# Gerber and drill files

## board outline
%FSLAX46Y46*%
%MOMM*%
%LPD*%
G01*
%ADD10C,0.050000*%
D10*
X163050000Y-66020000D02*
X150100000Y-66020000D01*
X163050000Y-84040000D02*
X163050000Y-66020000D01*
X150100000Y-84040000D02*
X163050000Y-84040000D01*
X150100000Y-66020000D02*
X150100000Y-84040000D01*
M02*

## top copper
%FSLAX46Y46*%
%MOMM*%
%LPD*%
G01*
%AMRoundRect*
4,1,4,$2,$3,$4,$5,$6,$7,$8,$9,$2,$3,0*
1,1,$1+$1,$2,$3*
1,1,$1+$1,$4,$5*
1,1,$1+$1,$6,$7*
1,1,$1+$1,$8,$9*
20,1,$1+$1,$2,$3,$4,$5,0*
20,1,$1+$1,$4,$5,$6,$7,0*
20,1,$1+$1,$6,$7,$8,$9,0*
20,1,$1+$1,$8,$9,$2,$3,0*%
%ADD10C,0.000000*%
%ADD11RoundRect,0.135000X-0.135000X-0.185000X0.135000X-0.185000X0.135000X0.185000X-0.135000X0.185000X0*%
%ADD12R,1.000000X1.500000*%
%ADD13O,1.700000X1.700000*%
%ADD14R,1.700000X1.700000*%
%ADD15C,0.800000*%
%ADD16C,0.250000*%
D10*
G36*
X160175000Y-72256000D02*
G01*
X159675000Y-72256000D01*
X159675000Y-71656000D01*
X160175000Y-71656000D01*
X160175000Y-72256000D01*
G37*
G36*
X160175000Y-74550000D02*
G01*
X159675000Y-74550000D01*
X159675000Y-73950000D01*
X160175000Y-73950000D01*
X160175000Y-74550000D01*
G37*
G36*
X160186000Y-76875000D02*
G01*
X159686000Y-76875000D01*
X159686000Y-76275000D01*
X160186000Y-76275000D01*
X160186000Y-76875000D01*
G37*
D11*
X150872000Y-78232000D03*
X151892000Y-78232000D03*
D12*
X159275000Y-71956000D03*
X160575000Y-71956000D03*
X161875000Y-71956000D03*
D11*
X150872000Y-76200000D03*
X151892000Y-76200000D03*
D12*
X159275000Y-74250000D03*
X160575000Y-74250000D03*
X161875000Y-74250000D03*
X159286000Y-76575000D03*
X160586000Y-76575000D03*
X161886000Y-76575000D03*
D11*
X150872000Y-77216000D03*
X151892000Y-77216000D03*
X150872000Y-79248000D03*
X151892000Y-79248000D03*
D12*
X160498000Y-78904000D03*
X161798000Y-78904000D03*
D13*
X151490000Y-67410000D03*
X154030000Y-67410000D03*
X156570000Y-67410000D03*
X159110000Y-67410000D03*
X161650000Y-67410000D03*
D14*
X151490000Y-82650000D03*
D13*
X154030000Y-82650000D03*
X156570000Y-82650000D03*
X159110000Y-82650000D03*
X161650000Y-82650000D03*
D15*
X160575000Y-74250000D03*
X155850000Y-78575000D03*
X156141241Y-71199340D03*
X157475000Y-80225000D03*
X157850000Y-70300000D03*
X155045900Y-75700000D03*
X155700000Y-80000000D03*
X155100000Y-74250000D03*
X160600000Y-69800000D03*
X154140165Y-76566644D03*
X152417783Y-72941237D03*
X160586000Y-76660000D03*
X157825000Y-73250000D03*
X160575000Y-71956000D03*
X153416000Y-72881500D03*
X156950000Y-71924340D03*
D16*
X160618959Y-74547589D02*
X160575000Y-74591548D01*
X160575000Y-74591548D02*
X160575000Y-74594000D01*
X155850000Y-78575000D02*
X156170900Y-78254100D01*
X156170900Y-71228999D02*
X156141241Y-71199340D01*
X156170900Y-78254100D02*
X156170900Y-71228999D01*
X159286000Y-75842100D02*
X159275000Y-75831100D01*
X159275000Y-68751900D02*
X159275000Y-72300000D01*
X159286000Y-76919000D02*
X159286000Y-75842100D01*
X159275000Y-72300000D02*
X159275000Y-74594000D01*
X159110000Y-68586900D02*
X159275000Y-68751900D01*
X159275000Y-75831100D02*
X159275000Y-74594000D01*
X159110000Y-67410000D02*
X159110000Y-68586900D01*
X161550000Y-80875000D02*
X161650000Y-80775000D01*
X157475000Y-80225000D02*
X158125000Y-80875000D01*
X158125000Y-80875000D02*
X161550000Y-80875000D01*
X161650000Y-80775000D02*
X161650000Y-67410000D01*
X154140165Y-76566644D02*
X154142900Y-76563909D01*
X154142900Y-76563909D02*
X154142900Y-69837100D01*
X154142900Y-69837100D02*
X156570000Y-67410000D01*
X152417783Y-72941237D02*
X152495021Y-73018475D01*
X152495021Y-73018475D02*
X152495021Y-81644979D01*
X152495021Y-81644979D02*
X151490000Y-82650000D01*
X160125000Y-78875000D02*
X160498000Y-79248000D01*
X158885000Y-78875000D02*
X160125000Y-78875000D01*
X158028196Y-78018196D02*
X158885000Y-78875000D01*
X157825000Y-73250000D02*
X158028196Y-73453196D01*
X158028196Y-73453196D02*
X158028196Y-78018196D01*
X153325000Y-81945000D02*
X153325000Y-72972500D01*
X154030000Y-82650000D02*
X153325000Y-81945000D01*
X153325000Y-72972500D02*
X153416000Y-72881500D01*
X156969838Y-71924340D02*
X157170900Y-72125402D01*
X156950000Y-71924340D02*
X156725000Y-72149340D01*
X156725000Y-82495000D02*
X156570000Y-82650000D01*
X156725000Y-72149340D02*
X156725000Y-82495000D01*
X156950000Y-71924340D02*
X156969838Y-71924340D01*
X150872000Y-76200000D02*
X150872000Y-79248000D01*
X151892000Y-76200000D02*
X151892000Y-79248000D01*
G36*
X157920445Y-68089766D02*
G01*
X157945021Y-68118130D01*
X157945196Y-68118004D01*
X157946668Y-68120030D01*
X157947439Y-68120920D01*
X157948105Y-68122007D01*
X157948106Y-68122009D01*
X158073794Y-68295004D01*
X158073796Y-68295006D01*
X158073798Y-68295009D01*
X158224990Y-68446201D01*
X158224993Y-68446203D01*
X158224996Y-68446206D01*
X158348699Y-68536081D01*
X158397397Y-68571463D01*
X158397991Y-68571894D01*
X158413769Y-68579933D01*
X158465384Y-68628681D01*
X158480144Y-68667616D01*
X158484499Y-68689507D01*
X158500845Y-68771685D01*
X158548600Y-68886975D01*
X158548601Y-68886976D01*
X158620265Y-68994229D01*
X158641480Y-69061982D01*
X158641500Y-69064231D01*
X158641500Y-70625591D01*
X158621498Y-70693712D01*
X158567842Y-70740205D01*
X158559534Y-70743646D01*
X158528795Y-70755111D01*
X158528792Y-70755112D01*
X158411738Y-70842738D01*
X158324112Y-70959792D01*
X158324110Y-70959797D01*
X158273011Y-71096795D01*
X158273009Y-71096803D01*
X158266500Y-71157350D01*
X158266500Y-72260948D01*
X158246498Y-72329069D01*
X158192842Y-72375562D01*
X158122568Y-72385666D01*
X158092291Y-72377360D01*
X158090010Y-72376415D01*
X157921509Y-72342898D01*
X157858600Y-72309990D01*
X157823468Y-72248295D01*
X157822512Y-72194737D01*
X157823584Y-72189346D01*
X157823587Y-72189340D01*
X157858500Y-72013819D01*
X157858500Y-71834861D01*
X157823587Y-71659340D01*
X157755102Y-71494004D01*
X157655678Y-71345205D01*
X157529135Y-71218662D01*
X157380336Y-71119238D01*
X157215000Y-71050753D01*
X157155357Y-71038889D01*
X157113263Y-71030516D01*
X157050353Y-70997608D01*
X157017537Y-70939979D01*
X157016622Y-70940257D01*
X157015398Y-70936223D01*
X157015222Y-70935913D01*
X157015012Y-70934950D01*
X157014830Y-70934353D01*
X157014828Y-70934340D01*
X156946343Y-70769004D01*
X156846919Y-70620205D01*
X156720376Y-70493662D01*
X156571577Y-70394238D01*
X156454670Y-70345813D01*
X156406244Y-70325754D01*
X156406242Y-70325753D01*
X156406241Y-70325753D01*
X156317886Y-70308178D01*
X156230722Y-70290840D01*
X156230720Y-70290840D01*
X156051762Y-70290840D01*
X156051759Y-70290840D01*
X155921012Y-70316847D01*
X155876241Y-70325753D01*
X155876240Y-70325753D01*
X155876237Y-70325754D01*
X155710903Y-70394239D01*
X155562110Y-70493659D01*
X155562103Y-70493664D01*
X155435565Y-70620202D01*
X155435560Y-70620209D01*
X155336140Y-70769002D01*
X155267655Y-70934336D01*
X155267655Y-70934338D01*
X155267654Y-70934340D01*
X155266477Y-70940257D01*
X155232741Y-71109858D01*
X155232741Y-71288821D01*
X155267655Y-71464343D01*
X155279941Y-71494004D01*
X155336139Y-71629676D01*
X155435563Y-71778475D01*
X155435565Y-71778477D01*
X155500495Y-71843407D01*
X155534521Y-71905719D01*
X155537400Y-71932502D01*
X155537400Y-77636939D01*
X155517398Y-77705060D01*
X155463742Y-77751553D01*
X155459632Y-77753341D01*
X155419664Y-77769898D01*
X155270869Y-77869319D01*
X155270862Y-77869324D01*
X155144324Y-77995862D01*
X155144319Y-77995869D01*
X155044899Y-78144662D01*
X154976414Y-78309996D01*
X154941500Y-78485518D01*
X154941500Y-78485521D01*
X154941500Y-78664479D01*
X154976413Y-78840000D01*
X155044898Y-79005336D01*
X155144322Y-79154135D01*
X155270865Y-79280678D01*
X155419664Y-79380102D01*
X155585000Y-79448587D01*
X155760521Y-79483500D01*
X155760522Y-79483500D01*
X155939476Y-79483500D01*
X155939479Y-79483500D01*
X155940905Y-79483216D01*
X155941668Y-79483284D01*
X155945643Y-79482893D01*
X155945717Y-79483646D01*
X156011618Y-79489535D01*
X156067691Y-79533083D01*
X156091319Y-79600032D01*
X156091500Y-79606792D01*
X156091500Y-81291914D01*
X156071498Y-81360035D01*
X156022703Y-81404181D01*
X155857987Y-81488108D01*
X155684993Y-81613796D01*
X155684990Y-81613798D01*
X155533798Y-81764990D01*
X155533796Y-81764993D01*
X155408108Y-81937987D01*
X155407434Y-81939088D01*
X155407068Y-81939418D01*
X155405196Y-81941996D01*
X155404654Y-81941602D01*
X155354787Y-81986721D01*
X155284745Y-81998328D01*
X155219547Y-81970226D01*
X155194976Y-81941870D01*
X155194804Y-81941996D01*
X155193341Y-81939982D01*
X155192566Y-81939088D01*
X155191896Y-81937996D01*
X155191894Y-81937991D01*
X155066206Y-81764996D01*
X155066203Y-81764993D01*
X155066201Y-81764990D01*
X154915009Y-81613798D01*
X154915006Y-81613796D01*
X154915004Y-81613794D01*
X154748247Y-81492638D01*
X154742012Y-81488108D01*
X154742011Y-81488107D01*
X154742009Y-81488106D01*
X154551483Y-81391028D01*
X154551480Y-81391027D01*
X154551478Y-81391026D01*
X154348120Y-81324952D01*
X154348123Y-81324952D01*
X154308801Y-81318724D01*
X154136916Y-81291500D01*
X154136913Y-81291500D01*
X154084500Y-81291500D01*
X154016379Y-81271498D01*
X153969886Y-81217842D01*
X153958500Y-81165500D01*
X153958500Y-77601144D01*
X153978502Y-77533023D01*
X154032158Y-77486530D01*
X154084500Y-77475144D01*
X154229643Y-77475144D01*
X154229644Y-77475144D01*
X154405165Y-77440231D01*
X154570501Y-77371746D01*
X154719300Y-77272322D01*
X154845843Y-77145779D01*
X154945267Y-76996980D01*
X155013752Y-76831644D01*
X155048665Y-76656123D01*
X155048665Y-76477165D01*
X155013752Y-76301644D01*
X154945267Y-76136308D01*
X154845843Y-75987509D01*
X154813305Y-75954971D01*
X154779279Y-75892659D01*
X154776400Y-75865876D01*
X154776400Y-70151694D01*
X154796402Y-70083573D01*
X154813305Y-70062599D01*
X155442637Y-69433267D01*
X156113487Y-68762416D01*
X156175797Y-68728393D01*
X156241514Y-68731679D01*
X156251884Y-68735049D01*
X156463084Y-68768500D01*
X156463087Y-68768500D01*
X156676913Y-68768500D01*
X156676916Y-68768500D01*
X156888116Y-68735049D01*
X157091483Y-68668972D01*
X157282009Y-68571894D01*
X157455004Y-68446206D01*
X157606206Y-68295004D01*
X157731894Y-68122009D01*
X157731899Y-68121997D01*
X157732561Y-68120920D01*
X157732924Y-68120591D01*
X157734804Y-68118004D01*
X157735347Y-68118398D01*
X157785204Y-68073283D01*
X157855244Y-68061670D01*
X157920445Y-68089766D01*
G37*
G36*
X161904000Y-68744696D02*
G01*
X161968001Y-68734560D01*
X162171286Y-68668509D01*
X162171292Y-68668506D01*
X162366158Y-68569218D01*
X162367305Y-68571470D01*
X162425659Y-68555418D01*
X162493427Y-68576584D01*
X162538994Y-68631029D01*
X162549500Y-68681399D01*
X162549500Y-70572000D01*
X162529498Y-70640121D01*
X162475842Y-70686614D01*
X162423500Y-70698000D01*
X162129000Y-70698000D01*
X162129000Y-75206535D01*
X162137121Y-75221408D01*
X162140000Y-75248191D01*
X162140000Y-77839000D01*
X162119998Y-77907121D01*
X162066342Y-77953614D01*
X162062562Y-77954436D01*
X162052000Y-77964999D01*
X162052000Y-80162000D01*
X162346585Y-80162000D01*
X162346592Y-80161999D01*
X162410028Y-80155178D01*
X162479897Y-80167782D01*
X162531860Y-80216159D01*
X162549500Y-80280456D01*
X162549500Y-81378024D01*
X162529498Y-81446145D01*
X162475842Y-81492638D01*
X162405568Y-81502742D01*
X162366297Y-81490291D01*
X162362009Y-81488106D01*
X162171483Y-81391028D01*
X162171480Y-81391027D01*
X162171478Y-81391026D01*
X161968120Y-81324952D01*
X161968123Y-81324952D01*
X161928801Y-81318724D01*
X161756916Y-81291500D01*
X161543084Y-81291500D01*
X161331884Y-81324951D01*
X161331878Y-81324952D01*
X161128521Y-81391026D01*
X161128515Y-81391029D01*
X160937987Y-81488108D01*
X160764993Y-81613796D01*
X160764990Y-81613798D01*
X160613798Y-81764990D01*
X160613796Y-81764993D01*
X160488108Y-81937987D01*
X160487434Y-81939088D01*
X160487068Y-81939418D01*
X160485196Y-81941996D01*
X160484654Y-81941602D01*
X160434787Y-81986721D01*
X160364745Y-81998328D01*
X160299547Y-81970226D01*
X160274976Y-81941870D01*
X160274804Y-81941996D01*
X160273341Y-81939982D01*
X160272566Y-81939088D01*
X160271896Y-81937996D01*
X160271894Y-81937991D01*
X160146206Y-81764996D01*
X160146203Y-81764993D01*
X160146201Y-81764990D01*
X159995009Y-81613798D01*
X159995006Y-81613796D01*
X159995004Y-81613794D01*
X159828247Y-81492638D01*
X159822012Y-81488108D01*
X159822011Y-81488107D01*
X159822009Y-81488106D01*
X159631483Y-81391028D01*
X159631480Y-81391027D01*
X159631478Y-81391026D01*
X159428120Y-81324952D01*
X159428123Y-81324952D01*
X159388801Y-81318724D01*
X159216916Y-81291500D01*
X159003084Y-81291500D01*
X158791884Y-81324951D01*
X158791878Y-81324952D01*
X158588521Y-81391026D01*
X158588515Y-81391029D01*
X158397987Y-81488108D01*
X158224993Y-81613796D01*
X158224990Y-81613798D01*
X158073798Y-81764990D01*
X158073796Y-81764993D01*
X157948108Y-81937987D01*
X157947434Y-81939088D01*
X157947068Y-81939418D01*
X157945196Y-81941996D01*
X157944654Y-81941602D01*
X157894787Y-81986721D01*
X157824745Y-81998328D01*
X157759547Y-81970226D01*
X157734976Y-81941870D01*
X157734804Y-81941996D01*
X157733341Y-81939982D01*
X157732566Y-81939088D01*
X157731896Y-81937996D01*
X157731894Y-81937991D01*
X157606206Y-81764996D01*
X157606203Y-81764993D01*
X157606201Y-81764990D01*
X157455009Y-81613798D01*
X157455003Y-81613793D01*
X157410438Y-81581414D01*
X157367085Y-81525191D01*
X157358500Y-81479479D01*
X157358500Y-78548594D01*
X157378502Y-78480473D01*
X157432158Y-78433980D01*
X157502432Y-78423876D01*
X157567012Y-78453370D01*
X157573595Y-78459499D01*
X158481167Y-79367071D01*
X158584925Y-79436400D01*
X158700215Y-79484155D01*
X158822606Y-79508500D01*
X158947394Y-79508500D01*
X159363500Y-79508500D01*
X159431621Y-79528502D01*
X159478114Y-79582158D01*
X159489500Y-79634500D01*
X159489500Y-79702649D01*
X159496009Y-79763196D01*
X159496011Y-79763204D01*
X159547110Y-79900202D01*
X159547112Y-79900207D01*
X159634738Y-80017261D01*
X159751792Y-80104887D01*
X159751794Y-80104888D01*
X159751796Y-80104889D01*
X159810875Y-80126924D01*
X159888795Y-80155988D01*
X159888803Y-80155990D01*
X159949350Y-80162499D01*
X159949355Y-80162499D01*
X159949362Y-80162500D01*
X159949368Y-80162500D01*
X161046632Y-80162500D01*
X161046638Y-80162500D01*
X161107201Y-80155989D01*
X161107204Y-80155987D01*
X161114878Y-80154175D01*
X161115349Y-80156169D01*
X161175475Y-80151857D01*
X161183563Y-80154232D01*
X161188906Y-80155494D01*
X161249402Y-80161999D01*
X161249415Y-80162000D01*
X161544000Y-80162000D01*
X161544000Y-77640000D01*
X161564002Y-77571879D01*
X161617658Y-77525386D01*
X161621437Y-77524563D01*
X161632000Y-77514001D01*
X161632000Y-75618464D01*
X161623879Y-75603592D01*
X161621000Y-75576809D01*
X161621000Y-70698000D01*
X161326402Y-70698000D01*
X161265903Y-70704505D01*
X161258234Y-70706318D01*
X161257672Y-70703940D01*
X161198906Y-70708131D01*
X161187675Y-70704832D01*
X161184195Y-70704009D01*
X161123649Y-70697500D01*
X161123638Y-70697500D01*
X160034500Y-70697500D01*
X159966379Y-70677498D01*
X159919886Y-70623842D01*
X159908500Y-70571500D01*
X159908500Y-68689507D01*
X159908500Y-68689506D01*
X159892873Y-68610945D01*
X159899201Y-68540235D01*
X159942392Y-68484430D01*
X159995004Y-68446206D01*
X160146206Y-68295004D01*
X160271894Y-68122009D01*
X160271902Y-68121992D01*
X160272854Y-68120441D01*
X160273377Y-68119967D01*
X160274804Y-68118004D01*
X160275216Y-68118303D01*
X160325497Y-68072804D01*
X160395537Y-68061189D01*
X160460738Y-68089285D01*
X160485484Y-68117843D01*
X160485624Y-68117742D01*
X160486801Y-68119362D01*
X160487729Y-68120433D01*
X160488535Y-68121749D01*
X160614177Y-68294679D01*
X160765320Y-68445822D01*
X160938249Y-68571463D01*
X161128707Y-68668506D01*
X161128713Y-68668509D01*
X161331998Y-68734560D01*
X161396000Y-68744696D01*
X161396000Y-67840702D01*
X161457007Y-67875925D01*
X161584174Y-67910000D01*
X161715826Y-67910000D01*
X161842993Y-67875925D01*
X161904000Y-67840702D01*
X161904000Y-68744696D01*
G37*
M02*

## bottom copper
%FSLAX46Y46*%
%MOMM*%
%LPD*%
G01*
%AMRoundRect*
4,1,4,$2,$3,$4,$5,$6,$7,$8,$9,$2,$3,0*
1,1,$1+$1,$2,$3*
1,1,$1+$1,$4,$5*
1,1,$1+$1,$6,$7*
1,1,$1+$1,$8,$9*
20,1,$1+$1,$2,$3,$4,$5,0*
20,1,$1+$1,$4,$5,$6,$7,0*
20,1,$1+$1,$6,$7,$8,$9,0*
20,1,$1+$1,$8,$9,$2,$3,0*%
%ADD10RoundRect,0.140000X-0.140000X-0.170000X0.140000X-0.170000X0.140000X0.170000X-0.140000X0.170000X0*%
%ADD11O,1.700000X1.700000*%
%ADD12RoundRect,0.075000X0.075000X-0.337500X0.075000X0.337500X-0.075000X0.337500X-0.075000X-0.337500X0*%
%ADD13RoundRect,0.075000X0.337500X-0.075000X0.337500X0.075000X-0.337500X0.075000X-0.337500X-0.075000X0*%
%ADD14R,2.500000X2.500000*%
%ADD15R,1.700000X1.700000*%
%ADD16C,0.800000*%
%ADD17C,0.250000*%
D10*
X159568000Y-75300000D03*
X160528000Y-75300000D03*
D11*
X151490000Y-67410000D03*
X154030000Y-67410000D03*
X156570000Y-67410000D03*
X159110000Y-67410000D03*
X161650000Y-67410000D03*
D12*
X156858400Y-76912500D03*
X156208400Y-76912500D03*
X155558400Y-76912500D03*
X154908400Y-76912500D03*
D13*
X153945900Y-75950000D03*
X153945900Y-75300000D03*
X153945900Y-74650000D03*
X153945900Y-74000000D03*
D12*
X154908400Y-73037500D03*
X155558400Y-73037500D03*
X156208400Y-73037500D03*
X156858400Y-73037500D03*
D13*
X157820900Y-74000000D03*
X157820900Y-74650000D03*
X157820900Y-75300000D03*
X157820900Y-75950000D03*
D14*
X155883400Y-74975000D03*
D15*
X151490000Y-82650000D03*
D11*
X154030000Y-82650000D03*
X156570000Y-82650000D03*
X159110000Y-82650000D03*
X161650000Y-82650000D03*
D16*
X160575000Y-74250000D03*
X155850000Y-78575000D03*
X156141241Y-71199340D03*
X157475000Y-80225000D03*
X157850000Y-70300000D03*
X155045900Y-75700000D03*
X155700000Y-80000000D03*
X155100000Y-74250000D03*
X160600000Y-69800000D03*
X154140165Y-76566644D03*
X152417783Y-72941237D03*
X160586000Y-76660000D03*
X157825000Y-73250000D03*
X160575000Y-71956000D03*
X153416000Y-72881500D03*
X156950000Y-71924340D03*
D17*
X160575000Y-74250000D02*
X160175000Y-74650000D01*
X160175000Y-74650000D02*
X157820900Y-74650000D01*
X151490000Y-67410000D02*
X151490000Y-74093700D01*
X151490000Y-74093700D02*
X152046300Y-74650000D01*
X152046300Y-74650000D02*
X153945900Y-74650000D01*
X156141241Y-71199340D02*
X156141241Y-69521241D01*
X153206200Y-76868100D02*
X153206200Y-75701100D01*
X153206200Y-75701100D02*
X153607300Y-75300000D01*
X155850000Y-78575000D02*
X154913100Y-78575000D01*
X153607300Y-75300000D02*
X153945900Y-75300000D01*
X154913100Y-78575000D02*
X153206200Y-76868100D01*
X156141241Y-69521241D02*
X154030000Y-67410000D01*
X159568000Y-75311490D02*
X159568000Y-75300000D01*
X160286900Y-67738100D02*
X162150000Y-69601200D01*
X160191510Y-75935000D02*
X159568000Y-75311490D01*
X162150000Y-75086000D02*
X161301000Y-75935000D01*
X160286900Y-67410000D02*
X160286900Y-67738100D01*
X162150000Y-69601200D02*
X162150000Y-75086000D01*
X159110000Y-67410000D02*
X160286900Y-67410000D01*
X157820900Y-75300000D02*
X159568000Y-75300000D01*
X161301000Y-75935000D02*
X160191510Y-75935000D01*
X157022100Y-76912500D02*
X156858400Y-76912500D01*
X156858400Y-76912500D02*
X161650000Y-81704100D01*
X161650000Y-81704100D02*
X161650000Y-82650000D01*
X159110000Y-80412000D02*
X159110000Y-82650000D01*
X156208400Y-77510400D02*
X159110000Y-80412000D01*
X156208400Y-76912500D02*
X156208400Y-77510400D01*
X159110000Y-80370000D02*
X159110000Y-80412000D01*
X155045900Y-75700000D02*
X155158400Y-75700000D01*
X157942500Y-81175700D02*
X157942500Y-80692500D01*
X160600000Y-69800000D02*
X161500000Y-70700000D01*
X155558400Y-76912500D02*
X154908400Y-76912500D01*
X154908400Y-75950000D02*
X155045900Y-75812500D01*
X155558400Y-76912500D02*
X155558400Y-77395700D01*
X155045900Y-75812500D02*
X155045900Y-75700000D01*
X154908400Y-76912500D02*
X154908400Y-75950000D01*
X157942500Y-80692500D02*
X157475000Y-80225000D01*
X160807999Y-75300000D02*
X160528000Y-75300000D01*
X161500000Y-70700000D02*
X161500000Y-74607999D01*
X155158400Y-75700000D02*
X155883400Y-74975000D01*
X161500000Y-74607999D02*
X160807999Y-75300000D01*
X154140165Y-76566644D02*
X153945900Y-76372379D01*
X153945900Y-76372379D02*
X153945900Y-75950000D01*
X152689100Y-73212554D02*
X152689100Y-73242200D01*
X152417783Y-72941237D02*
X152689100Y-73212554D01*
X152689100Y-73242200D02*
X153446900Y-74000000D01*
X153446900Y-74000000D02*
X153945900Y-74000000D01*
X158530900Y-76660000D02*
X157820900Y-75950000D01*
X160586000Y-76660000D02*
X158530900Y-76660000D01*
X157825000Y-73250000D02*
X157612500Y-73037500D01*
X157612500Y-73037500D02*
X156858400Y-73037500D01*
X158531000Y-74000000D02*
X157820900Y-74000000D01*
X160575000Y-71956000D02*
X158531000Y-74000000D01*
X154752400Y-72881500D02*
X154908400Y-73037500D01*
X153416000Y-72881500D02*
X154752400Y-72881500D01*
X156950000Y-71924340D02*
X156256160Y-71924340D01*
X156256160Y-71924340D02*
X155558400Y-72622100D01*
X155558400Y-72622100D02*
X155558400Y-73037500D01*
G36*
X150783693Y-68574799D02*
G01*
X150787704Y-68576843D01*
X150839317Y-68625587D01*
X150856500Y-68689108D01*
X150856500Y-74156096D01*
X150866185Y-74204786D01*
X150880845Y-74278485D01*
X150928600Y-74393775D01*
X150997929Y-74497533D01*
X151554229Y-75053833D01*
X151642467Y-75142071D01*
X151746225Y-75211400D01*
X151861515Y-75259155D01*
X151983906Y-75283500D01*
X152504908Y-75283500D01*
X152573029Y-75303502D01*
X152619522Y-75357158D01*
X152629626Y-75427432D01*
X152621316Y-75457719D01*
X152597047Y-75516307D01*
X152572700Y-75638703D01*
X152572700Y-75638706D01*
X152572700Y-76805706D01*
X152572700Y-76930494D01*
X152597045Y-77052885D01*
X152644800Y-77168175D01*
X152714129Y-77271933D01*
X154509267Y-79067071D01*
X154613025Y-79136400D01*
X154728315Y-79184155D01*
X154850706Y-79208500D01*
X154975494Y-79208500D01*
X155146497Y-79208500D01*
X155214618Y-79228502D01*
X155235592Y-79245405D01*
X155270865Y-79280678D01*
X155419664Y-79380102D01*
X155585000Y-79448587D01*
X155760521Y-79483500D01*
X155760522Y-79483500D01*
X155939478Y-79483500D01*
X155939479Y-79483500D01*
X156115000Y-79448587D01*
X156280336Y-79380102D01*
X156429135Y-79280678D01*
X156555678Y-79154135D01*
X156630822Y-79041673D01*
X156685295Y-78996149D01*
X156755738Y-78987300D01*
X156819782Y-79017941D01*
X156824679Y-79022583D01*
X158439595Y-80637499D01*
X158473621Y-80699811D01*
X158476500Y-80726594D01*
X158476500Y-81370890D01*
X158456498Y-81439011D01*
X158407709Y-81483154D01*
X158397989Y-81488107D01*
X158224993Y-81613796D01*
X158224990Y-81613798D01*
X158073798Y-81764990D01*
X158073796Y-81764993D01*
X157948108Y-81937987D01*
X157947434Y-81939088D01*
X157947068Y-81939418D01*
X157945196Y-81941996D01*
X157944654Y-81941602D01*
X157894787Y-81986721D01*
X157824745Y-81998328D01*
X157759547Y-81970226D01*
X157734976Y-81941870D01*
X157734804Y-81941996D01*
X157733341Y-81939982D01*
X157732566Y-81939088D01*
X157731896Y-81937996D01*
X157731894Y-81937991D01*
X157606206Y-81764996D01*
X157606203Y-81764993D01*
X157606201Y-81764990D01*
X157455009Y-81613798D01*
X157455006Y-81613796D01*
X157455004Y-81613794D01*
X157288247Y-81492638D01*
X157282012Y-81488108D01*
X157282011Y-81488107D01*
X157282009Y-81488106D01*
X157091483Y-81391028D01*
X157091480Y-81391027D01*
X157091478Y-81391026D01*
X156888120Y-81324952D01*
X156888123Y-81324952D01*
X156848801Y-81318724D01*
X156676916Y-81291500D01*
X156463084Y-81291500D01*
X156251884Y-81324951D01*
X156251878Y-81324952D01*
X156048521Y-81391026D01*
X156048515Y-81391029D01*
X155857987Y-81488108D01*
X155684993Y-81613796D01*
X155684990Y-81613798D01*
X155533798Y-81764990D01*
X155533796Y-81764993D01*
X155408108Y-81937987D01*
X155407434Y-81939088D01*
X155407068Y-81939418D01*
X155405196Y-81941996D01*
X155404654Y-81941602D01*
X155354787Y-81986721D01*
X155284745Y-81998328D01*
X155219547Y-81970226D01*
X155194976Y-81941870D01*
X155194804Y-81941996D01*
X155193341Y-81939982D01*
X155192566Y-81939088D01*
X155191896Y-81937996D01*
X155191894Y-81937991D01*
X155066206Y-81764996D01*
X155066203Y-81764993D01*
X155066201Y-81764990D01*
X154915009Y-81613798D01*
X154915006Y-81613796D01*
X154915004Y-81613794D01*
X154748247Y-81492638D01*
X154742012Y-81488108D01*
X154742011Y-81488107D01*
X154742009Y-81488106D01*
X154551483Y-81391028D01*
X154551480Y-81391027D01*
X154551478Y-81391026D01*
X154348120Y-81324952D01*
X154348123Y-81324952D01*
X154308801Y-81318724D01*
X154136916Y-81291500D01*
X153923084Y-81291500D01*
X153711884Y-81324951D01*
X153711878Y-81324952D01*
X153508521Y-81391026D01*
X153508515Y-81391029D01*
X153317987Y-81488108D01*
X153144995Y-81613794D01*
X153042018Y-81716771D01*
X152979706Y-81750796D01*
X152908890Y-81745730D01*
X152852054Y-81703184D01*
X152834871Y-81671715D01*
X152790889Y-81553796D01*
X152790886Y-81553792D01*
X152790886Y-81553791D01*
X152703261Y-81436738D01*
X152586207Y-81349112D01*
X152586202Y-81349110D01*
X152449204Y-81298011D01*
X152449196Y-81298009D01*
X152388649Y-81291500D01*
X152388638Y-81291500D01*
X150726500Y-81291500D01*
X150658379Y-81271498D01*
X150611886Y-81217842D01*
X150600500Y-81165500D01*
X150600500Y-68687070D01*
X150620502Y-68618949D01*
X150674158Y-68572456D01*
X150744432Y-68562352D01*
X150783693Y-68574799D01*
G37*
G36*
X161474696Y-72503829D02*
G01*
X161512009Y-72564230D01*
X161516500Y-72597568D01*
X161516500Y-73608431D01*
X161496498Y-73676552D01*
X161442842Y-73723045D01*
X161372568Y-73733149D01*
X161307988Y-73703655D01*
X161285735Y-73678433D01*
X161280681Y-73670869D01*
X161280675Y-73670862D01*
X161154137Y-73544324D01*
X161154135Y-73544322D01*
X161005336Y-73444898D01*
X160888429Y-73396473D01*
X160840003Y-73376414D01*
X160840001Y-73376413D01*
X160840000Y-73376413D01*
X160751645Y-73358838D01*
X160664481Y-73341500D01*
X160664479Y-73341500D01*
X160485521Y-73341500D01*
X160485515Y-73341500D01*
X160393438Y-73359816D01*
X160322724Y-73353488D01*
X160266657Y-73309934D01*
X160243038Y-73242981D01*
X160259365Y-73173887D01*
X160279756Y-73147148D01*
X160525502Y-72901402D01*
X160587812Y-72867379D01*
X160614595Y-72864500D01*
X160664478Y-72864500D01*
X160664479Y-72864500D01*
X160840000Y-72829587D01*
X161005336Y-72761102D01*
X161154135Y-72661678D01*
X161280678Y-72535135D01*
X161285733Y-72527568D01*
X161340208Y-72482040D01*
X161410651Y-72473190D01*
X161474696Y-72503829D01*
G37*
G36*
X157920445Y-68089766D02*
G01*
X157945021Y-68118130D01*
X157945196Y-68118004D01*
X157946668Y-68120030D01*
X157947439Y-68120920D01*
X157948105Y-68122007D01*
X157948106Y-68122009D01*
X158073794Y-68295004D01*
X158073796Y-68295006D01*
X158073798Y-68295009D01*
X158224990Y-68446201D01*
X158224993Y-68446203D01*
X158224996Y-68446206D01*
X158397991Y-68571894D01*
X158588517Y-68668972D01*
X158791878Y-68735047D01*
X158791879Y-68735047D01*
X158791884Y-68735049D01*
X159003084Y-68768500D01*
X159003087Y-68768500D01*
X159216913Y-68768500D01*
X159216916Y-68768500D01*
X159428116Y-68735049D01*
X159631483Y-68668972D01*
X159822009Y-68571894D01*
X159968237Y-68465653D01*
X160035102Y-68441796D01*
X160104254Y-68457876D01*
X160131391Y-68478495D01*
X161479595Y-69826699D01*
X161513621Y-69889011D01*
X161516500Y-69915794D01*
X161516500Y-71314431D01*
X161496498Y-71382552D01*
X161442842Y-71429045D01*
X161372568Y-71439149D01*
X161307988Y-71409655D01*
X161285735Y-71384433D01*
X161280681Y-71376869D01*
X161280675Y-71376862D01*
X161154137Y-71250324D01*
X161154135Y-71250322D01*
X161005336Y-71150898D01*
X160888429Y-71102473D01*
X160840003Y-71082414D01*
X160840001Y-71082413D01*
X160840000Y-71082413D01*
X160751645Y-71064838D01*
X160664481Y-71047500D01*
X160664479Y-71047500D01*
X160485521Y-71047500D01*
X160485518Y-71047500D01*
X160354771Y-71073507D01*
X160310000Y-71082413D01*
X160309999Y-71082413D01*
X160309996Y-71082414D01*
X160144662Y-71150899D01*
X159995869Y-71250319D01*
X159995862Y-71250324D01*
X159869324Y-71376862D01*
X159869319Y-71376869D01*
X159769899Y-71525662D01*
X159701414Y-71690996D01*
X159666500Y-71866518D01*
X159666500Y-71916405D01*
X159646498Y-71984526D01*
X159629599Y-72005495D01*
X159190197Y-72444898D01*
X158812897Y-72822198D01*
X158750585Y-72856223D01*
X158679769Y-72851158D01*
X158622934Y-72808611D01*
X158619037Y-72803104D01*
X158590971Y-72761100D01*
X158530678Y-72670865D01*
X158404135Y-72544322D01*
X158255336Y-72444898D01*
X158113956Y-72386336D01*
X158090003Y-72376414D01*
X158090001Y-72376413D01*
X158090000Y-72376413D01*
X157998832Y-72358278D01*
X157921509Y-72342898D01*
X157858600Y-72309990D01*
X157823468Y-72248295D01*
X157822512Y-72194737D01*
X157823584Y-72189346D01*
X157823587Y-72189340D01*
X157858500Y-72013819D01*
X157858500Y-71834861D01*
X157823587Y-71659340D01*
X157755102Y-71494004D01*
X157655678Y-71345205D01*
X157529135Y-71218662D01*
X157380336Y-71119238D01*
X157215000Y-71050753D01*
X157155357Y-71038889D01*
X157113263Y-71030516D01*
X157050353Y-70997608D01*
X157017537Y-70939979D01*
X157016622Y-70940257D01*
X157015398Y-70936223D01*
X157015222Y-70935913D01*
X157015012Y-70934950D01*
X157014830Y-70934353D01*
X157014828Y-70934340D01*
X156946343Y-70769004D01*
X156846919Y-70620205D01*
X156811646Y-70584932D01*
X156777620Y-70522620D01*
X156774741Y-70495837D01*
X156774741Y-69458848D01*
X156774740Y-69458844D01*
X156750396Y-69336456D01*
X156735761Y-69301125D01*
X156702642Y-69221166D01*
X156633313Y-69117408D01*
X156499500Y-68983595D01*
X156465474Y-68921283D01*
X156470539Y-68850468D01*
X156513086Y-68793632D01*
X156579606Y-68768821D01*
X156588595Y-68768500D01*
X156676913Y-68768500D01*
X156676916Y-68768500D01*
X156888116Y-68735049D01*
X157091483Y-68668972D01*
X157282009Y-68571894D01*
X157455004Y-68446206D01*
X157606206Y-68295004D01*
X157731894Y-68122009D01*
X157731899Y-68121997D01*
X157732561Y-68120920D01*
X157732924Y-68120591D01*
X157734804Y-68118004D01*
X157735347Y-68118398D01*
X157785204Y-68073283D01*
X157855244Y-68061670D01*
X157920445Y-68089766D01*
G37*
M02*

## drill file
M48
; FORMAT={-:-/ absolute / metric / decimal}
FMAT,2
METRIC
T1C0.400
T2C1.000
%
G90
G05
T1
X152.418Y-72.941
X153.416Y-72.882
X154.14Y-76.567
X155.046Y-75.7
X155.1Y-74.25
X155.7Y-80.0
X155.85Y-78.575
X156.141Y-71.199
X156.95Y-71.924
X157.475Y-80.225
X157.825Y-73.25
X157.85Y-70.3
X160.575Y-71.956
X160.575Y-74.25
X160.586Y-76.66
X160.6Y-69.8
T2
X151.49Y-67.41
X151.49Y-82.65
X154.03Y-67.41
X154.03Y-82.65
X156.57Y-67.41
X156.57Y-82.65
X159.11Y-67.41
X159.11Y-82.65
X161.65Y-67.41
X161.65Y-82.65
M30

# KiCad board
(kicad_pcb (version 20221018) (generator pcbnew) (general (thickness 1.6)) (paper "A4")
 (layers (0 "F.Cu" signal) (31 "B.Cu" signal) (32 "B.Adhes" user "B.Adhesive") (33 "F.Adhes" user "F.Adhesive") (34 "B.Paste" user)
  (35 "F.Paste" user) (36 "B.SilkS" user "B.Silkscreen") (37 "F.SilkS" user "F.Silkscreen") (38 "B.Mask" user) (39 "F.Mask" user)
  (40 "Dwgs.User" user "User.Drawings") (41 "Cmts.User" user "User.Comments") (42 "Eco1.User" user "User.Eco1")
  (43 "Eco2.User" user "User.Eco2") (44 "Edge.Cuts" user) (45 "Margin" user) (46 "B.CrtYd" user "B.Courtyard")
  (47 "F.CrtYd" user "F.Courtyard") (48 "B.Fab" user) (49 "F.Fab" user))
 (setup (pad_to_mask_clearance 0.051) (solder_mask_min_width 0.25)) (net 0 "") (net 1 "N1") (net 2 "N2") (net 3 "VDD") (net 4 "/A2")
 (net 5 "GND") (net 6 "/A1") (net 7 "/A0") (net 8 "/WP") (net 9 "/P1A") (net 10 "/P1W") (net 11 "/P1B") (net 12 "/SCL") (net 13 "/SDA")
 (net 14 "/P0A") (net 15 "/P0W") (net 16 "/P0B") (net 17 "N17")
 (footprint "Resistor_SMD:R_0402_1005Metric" (layer "F.Cu") (at 151.382 78.232)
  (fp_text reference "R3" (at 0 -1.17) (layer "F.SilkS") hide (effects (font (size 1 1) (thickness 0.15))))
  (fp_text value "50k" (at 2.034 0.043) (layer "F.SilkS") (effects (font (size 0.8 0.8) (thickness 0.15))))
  (pad "1" smd roundrect (at -0.51 0) (size 0.54 0.64) (layers "F.Cu" "F.Paste" "F.Mask") (roundrect_rratio 0.25) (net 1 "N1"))
  (pad "2" smd roundrect (at 0.51 0) (size 0.54 0.64) (layers "F.Cu" "F.Paste" "F.Mask") (roundrect_rratio 0.25) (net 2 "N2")))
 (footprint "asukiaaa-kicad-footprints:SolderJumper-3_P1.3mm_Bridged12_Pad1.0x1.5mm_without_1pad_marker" (layer "F.Cu") (at 160.575 71.956)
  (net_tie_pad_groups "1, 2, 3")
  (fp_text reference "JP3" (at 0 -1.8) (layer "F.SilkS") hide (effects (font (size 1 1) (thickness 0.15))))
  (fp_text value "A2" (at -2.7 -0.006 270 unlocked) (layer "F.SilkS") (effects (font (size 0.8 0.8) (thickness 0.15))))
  (fp_poly (pts (xy -0.9 -0.3) (xy -0.4 -0.3) (xy -0.4 0.3) (xy -0.9 0.3)) (stroke (width 0) (type solid)) (fill solid) (layer "F.Cu"))
  (pad "1" smd rect (at -1.3 0) (size 1 1.5) (layers "F.Cu" "F.Mask") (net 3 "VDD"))
  (pad "2" smd rect (at 0 0) (size 1 1.5) (layers "F.Cu" "F.Mask") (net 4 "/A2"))
  (pad "3" smd rect (at 1.3 0) (size 1 1.5) (layers "F.Cu" "F.Mask") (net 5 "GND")))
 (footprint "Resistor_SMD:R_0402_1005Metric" (layer "F.Cu") (at 151.382 76.2)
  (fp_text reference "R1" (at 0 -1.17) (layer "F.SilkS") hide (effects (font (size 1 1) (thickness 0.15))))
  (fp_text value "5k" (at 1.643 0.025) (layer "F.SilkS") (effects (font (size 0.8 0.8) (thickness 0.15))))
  (pad "1" smd roundrect (at -0.51 0) (size 0.54 0.64) (layers "F.Cu" "F.Paste" "F.Mask") (roundrect_rratio 0.25) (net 1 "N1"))
  (pad "2" smd roundrect (at 0.51 0) (size 0.54 0.64) (layers "F.Cu" "F.Paste" "F.Mask") (roundrect_rratio 0.25) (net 2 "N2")))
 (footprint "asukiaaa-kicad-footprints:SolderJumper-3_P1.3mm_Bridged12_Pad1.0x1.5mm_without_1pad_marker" (layer "F.Cu") (at 160.575 74.25)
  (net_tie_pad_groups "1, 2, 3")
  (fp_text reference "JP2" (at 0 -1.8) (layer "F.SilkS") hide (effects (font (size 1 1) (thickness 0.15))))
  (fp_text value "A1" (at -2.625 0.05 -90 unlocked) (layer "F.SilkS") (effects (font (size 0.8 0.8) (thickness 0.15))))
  (fp_poly (pts (xy -0.9 -0.3) (xy -0.4 -0.3) (xy -0.4 0.3) (xy -0.9 0.3)) (stroke (width 0) (type solid)) (fill solid) (layer "F.Cu"))
  (pad "1" smd rect (at -1.3 0) (size 1 1.5) (layers "F.Cu" "F.Mask") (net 3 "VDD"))
  (pad "2" smd rect (at 0 0) (size 1 1.5) (layers "F.Cu" "F.Mask") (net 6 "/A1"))
  (pad "3" smd rect (at 1.3 0) (size 1 1.5) (layers "F.Cu" "F.Mask") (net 5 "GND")))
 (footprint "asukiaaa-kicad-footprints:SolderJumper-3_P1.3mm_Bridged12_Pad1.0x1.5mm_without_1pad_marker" (layer "F.Cu") (at 160.586 76.575)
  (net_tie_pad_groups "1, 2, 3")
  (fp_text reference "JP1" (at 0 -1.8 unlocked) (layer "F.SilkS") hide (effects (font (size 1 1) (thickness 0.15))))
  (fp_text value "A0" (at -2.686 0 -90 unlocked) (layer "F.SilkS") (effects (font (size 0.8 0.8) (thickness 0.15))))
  (fp_poly (pts (xy -0.9 -0.3) (xy -0.4 -0.3) (xy -0.4 0.3) (xy -0.9 0.3)) (stroke (width 0) (type solid)) (fill solid) (layer "F.Cu"))
  (pad "1" smd rect (at -1.3 0) (size 1 1.5) (layers "F.Cu" "F.Mask") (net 3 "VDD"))
  (pad "2" smd rect (at 0 0) (size 1 1.5) (layers "F.Cu" "F.Mask") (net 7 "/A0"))
  (pad "3" smd rect (at 1.3 0) (size 1 1.5) (layers "F.Cu" "F.Mask") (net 5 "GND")))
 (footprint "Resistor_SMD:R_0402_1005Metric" (layer "F.Cu") (at 151.382 77.216)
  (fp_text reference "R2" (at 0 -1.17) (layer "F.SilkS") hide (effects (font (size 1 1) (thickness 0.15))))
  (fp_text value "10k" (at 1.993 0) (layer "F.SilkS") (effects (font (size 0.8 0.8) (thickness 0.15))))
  (pad "1" smd roundrect (at -0.51 0) (size 0.54 0.64) (layers "F.Cu" "F.Paste" "F.Mask") (roundrect_rratio 0.25) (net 1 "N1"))
  (pad "2" smd roundrect (at 0.51 0) (size 0.54 0.64) (layers "F.Cu" "F.Paste" "F.Mask") (roundrect_rratio 0.25) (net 2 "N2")))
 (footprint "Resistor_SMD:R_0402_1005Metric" (layer "F.Cu") (at 151.382 79.248)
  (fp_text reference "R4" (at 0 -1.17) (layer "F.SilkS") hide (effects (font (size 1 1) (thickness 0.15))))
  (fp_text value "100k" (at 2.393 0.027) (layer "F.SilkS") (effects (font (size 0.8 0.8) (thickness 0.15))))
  (pad "1" smd roundrect (at -0.51 0) (size 0.54 0.64) (layers "F.Cu" "F.Paste" "F.Mask") (roundrect_rratio 0.25) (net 1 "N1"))
  (pad "2" smd roundrect (at 0.51 0) (size 0.54 0.64) (layers "F.Cu" "F.Paste" "F.Mask") (roundrect_rratio 0.25) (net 2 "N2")))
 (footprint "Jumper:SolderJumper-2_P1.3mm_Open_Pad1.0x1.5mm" (layer "F.Cu") (at 161.148 78.904)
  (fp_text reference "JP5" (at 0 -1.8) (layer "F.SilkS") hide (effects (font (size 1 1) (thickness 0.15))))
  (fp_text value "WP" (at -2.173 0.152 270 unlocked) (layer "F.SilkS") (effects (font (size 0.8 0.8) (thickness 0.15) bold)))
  (pad "1" smd rect (at -0.65 0) (size 1 1.5) (layers "F.Cu" "F.Mask") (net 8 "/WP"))
  (pad "2" smd rect (at 0.65 0) (size 1 1.5) (layers "F.Cu" "F.Mask") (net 5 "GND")))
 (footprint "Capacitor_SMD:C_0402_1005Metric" (layer "B.Cu") (at 160.048 75.3)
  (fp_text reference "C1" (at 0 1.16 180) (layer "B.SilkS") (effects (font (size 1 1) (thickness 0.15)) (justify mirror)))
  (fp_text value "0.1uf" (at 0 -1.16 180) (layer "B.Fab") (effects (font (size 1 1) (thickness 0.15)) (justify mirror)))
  (pad "1" smd roundrect (at -0.48 0) (size 0.56 0.62) (layers "B.Cu" "B.Paste" "B.Mask") (roundrect_rratio 0.25) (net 3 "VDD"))
  (pad "2" smd roundrect (at 0.48 0) (size 0.56 0.62) (layers "B.Cu" "B.Paste" "B.Mask") (roundrect_rratio 0.25) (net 5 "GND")))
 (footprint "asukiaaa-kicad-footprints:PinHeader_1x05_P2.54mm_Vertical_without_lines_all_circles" (layer "B.Cu") (at 151.49 67.41 -90)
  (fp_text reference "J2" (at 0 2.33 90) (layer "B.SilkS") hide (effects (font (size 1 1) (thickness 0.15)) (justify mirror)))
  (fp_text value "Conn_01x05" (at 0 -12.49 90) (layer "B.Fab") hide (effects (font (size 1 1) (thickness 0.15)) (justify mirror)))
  (pad "1" thru_hole oval (at 0 0 270) (size 1.7 1.7) (drill 1) (layers "*.Cu" "*.Mask") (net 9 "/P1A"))
  (pad "2" thru_hole oval (at 0 -2.54 270) (size 1.7 1.7) (drill 1) (layers "*.Cu" "*.Mask") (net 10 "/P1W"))
  (pad "3" thru_hole oval (at 0 -5.08 270) (size 1.7 1.7) (drill 1) (layers "*.Cu" "*.Mask") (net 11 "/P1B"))
  (pad "4" thru_hole oval (at 0 -7.62 270) (size 1.7 1.7) (drill 1) (layers "*.Cu" "*.Mask") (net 3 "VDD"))
  (pad "5" thru_hole oval (at 0 -10.16 270) (size 1.7 1.7) (drill 1) (layers "*.Cu" "*.Mask") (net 5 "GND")))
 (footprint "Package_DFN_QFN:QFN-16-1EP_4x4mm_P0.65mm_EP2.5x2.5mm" (layer "B.Cu") (at 155.8834 74.975 90)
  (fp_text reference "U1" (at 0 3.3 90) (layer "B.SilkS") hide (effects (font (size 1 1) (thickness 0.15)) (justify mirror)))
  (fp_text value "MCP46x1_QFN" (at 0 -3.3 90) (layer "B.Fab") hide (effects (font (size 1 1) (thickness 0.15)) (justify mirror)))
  (pad "" smd roundrect (at -0.625 -0.625 90) (size 1.01 1.01) (layers "B.Paste") (roundrect_rratio 0.247525))
  (pad "" smd roundrect (at -0.625 0.625 90) (size 1.01 1.01) (layers "B.Paste") (roundrect_rratio 0.247525))
  (pad "" smd roundrect (at 0.625 -0.625 90) (size 1.01 1.01) (layers "B.Paste") (roundrect_rratio 0.247525))
  (pad "" smd roundrect (at 0.625 0.625 90) (size 1.01 1.01) (layers "B.Paste") (roundrect_rratio 0.247525))
  (pad "1" smd roundrect (at -1.9375 0.975 90) (size 0.825 0.3) (layers "B.Cu" "B.Paste" "B.Mask") (roundrect_rratio 0.25) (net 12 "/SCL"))
  (pad "2" smd roundrect (at -1.9375 0.325 90) (size 0.825 0.3) (layers "B.Cu" "B.Paste" "B.Mask") (roundrect_rratio 0.25) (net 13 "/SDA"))
  (pad "3" smd roundrect (at -1.9375 -0.325 90) (size 0.825 0.3) (layers "B.Cu" "B.Paste" "B.Mask") (roundrect_rratio 0.25) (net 5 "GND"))
  (pad "4" smd roundrect (at -1.9375 -0.975 90) (size 0.825 0.3) (layers "B.Cu" "B.Paste" "B.Mask") (roundrect_rratio 0.25) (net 5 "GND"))
  (pad "5" smd roundrect (at -0.975 -1.9375 90) (size 0.3 0.825) (layers "B.Cu" "B.Paste" "B.Mask") (roundrect_rratio 0.25) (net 11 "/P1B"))
  (pad "6" smd roundrect (at -0.325 -1.9375 90) (size 0.3 0.825) (layers "B.Cu" "B.Paste" "B.Mask") (roundrect_rratio 0.25) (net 10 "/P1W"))
  (pad "7" smd roundrect (at 0.325 -1.9375 90) (size 0.3 0.825) (layers "B.Cu" "B.Paste" "B.Mask") (roundrect_rratio 0.25) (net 9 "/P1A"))
  (pad "8" smd roundrect (at 0.975 -1.9375 90) (size 0.3 0.825) (layers "B.Cu" "B.Paste" "B.Mask") (roundrect_rratio 0.25) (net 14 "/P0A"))
  (pad "9" smd roundrect (at 1.9375 -0.975 90) (size 0.825 0.3) (layers "B.Cu" "B.Paste" "B.Mask") (roundrect_rratio 0.25) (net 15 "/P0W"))
  (pad "10" smd roundrect (at 1.9375 -0.325 90) (size 0.825 0.3) (layers "B.Cu" "B.Paste" "B.Mask") (roundrect_rratio 0.25) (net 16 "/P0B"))
  (pad "11" smd roundrect (at 1.9375 0.325 90) (size 0.825 0.3) (layers "B.Cu" "B.Paste" "B.Mask") (roundrect_rratio 0.25) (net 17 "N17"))
  (pad "12" smd roundrect (at 1.9375 0.975 90) (size 0.825 0.3) (layers "B.Cu" "B.Paste" "B.Mask") (roundrect_rratio 0.25) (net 8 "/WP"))
  (pad "13" smd roundrect (at 0.975 1.9375 90) (size 0.3 0.825) (layers "B.Cu" "B.Paste" "B.Mask") (roundrect_rratio 0.25) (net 4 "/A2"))
  (pad "14" smd roundrect (at 0.325 1.9375 90) (size 0.3 0.825) (layers "B.Cu" "B.Paste" "B.Mask") (roundrect_rratio 0.25) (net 6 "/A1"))
  (pad "15" smd roundrect (at -0.325 1.9375 90) (size 0.3 0.825) (layers "B.Cu" "B.Paste" "B.Mask") (roundrect_rratio 0.25) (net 3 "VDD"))
  (pad "16" smd roundrect (at -0.975 1.9375 90) (size 0.3 0.825) (layers "B.Cu" "B.Paste" "B.Mask") (roundrect_rratio 0.25) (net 7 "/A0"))
  (pad "17" smd rect (at 0 0 90) (size 2.5 2.5) (layers "B.Cu" "B.Mask") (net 5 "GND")))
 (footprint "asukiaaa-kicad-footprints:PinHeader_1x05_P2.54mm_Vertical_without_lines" (layer "B.Cu") (at 151.49 82.65 -90)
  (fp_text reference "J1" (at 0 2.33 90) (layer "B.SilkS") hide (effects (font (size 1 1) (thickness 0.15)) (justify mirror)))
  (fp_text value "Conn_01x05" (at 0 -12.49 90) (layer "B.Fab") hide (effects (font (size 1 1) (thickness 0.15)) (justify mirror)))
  (pad "1" thru_hole rect (at 0 0 270) (size 1.7 1.7) (drill 1) (layers "*.Cu" "*.Mask") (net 14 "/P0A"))
  (pad "2" thru_hole oval (at 0 -2.54 270) (size 1.7 1.7) (drill 1) (layers "*.Cu" "*.Mask") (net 15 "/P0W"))
  (pad "3" thru_hole oval (at 0 -5.08 270) (size 1.7 1.7) (drill 1) (layers "*.Cu" "*.Mask") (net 16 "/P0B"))
  (pad "4" thru_hole oval (at 0 -7.62 270) (size 1.7 1.7) (drill 1) (layers "*.Cu" "*.Mask") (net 13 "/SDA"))
  (pad "5" thru_hole oval (at 0 -10.16 270) (size 1.7 1.7) (drill 1) (layers "*.Cu" "*.Mask") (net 12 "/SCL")))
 (gr_line (start 163.05 66.02) (end 150.1 66.02) (stroke (width 0.05) (type solid)) (layer "Edge.Cuts"))
 (gr_line (start 163.05 84.04) (end 163.05 66.02) (stroke (width 0.05) (type solid)) (layer "Edge.Cuts"))
 (gr_line (start 150.1 84.04) (end 163.05 84.04) (stroke (width 0.05) (type solid)) (layer "Edge.Cuts"))
 (gr_line (start 150.1 66.02) (end 150.1 84.04) (stroke (width 0.05) (type solid)) (layer "Edge.Cuts"))
 (segment (start 160.618959 74.547589) (end 160.575 74.591548) (width 0.25) (layer "F.Cu") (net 6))
 (segment (start 160.575 74.591548) (end 160.575 74.594) (width 0.25) (layer "F.Cu") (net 6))
 (via (at 160.575 74.25) (size 0.8) (drill 0.4) (layers "F.Cu" "B.Cu") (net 6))
 (segment (start 160.575 74.25) (end 160.175 74.65) (width 0.25) (layer "B.Cu") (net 6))
 (segment (start 160.175 74.65) (end 157.8209 74.65) (width 0.25) (layer "B.Cu") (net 6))
 (segment (start 151.49 67.41) (end 151.49 74.0937) (width 0.25) (layer "B.Cu") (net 9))
 (segment (start 151.49 74.0937) (end 152.0463 74.65) (width 0.25) (layer "B.Cu") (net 9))
 (segment (start 152.0463 74.65) (end 153.9459 74.65) (width 0.25) (layer "B.Cu") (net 9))
 (segment (start 155.85 78.575) (end 156.1709 78.2541) (width 0.25) (layer "F.Cu") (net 10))
 (segment (start 156.1709 71.228999) (end 156.141241 71.19934) (width 0.25) (layer "F.Cu") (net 10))
 (segment (start 156.1709 78.2541) (end 156.1709 71.228999) (width 0.25) (layer "F.Cu") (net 10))
 (via (at 155.85 78.575) (size 0.8) (drill 0.4) (layers "F.Cu" "B.Cu") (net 10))
 (via (at 156.141241 71.19934) (size 0.8) (drill 0.4) (layers "F.Cu" "B.Cu") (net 10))
 (segment (start 156.141241 71.19934) (end 156.141241 69.521241) (width 0.25) (layer "B.Cu") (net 10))
 (segment (start 153.2062 76.8681) (end 153.2062 75.7011) (width 0.25) (layer "B.Cu") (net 10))
 (segment (start 153.2062 75.7011) (end 153.6073 75.3) (width 0.25) (layer "B.Cu") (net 10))
 (segment (start 155.85 78.575) (end 154.9131 78.575) (width 0.25) (layer "B.Cu") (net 10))
 (segment (start 153.6073 75.3) (end 153.9459 75.3) (width 0.25) (layer "B.Cu") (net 10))
 (segment (start 154.9131 78.575) (end 153.2062 76.8681) (width 0.25) (layer "B.Cu") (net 10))
 (segment (start 156.141241 69.521241) (end 154.03 67.41) (width 0.25) (layer "B.Cu") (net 10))
 (segment (start 159.286 75.8421) (end 159.275 75.8311) (width 0.25) (layer "F.Cu") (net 3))
 (segment (start 159.275 68.7519) (end 159.275 72.3) (width 0.25) (layer "F.Cu") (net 3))
 (segment (start 159.286 76.919) (end 159.286 75.8421) (width 0.25) (layer "F.Cu") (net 3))
 (segment (start 159.275 72.3) (end 159.275 74.594) (width 0.25) (layer "F.Cu") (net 3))
 (segment (start 159.11 68.5869) (end 159.275 68.7519) (width 0.25) (layer "F.Cu") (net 3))
 (segment (start 159.275 75.8311) (end 159.275 74.594) (width 0.25) (layer "F.Cu") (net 3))
 (segment (start 159.11 67.41) (end 159.11 68.5869) (width 0.25) (layer "F.Cu") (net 3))
 (segment (start 159.568 75.31149) (end 159.568 75.3) (width 0.25) (layer "B.Cu") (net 3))
 (segment (start 160.2869 67.7381) (end 162.15 69.6012) (width 0.25) (layer "B.Cu") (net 3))
 (segment (start 160.19151 75.935) (end 159.568 75.31149) (width 0.25) (layer "B.Cu") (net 3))
 (segment (start 162.15 75.086) (end 161.301 75.935) (width 0.25) (layer "B.Cu") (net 3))
 (segment (start 160.2869 67.41) (end 160.2869 67.7381) (width 0.25) (layer "B.Cu") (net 3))
 (segment (start 162.15 69.6012) (end 162.15 75.086) (width 0.25) (layer "B.Cu") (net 3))
 (segment (start 159.11 67.41) (end 160.2869 67.41) (width 0.25) (layer "B.Cu") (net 3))
 (segment (start 157.8209 75.3) (end 159.568 75.3) (width 0.25) (layer "B.Cu") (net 3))
 (segment (start 161.301 75.935) (end 160.19151 75.935) (width 0.25) (layer "B.Cu") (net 3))
 (segment (start 157.0221 76.9125) (end 156.8584 76.9125) (width 0.25) (layer "B.Cu") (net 12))
 (segment (start 156.8584 76.9125) (end 161.65 81.7041) (width 0.25) (layer "B.Cu") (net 12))
 (segment (start 161.65 81.7041) (end 161.65 82.65) (width 0.25) (layer "B.Cu") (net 12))
 (segment (start 159.11 80.412) (end 159.11 82.65) (width 0.25) (layer "B.Cu") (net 13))
 (segment (start 156.2084 77.5104) (end 159.11 80.412) (width 0.25) (layer "B.Cu") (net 13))
 (segment (start 156.2084 76.9125) (end 156.2084 77.5104) (width 0.25) (layer "B.Cu") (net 13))
 (segment (start 159.11 80.37) (end 159.11 80.412) (width 0.25) (layer "B.Cu") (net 13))
 (segment (start 161.55 80.875) (end 161.65 80.775) (width 0.25) (layer "F.Cu") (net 5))
 (segment (start 157.475 80.225) (end 158.125 80.875) (width 0.25) (layer "F.Cu") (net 5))
 (segment (start 158.125 80.875) (end 161.55 80.875) (width 0.25) (layer "F.Cu") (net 5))
 (segment (start 161.65 80.775) (end 161.65 67.41) (width 0.25) (layer "F.Cu") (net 5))
 (via (at 157.475 80.225) (size 0.8) (drill 0.4) (layers "F.Cu" "B.Cu") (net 5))
 (via (at 157.85 70.3) (size 0.8) (drill 0.4) (layers "F.Cu" "B.Cu") (free) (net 5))
 (via (at 155.0459 75.7) (size 0.8) (drill 0.4) (layers "F.Cu" "B.Cu") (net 5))
 (via (at 155.7 80) (size 0.8) (drill 0.4) (layers "F.Cu" "B.Cu") (free) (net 5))
 (via (at 155.1 74.25) (size 0.8) (drill 0.4) (layers "F.Cu" "B.Cu") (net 5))
 (via (at 160.6 69.8) (size 0.8) (drill 0.4) (layers "F.Cu" "B.Cu") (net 5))
 (segment (start 155.0459 75.7) (end 155.1584 75.7) (width 0.25) (layer "B.Cu") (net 5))
 (segment (start 157.9425 81.1757) (end 157.9425 80.6925) (width 0.25) (layer "B.Cu") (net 5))
 (segment (start 160.6 69.8) (end 161.5 70.7) (width 0.25) (layer "B.Cu") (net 5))
 (segment (start 155.5584 76.9125) (end 154.9084 76.9125) (width 0.25) (layer "B.Cu") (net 5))
 (segment (start 154.9084 75.95) (end 155.0459 75.8125) (width 0.25) (layer "B.Cu") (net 5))
 (segment (start 155.5584 76.9125) (end 155.5584 77.3957) (width 0.25) (layer "B.Cu") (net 5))
 (segment (start 155.0459 75.8125) (end 155.0459 75.7) (width 0.25) (layer "B.Cu") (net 5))
 (segment (start 154.9084 76.9125) (end 154.9084 75.95) (width 0.25) (layer "B.Cu") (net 5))
 (segment (start 157.9425 80.6925) (end 157.475 80.225) (width 0.25) (layer "B.Cu") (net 5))
 (segment (start 160.807999 75.3) (end 160.528 75.3) (width 0.25) (layer "B.Cu") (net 5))
 (segment (start 161.5 70.7) (end 161.5 74.607999) (width 0.25) (layer "B.Cu") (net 5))
 (segment (start 155.1584 75.7) (end 155.8834 74.975) (width 0.25) (layer "B.Cu") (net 5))
 (segment (start 161.5 74.607999) (end 160.807999 75.3) (width 0.25) (layer "B.Cu") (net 5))
 (segment (start 154.140165 76.566644) (end 154.1429 76.563909) (width 0.25) (layer "F.Cu") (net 11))
 (segment (start 154.1429 76.563909) (end 154.1429 69.8371) (width 0.25) (layer "F.Cu") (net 11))
 (segment (start 154.1429 69.8371) (end 156.57 67.41) (width 0.25) (layer "F.Cu") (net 11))
 (via (at 154.140165 76.566644) (size 0.8) (drill 0.4) (layers "F.Cu" "B.Cu") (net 11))
 (segment (start 154.140165 76.566644) (end 153.9459 76.372379) (width 0.25) (layer "B.Cu") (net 11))
 (segment (start 153.9459 76.372379) (end 153.9459 75.95) (width 0.25) (layer "B.Cu") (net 11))
 (segment (start 152.417783 72.941237) (end 152.495021 73.018475) (width 0.25) (layer "F.Cu") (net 14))
 (segment (start 152.495021 73.018475) (end 152.495021 81.644979) (width 0.25) (layer "F.Cu") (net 14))
 (segment (start 152.495021 81.644979) (end 151.49 82.65) (width 0.25) (layer "F.Cu") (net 14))
 (via (at 152.417783 72.941237) (size 0.8) (drill 0.4) (layers "F.Cu" "B.Cu") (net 14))
 (segment (start 152.6891 73.212554) (end 152.6891 73.2422) (width 0.25) (layer "B.Cu") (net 14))
 (segment (start 152.417783 72.941237) (end 152.6891 73.212554) (width 0.25) (layer "B.Cu") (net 14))
 (segment (start 152.6891 73.2422) (end 153.4469 74) (width 0.25) (layer "B.Cu") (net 14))
 (segment (start 153.4469 74) (end 153.9459 74) (width 0.25) (layer "B.Cu") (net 14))
 (via (at 160.586 76.66) (size 0.8) (drill 0.4) (layers "F.Cu" "B.Cu") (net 7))
 (segment (start 158.5309 76.66) (end 157.8209 75.95) (width 0.25) (layer "B.Cu") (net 7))
 (segment (start 160.586 76.66) (end 158.5309 76.66) (width 0.25) (layer "B.Cu") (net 7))
 (segment (start 160.125 78.875) (end 160.498 79.248) (width 0.25) (layer "F.Cu") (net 8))
 (segment (start 158.885 78.875) (end 160.125 78.875) (width 0.25) (layer "F.Cu") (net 8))
 (segment (start 158.028196 78.018196) (end 158.885 78.875) (width 0.25) (layer "F.Cu") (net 8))
 (segment (start 157.825 73.25) (end 158.028196 73.453196) (width 0.25) (layer "F.Cu") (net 8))
 (segment (start 158.028196 73.453196) (end 158.028196 78.018196) (width 0.25) (layer "F.Cu") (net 8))
 (via (at 157.825 73.25) (size 0.8) (drill 0.4) (layers "F.Cu" "B.Cu") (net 8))
 (segment (start 157.825 73.25) (end 157.6125 73.0375) (width 0.25) (layer "B.Cu") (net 8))
 (segment (start 157.6125 73.0375) (end 156.8584 73.0375) (width 0.25) (layer "B.Cu") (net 8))
 (via (at 160.575 71.956) (size 0.8) (drill 0.4) (layers "F.Cu" "B.Cu") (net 4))
 (segment (start 158.531 74) (end 157.8209 74) (width 0.25) (layer "B.Cu") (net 4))
 (segment (start 160.575 71.956) (end 158.531 74) (width 0.25) (layer "B.Cu") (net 4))
 (segment (start 153.325 81.945) (end 153.325 72.9725) (width 0.25) (layer "F.Cu") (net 15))
 (segment (start 154.03 82.65) (end 153.325 81.945) (width 0.25) (layer "F.Cu") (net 15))
 (segment (start 153.325 72.9725) (end 153.416 72.8815) (width 0.25) (layer "F.Cu") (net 15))
 (via (at 153.416 72.8815) (size 0.8) (drill 0.4) (layers "F.Cu" "B.Cu") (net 15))
 (segment (start 154.7524 72.8815) (end 154.9084 73.0375) (width 0.25) (layer "B.Cu") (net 15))
 (segment (start 153.416 72.8815) (end 154.7524 72.8815) (width 0.25) (layer "B.Cu") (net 15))
 (segment (start 156.969838 71.92434) (end 157.1709 72.125402) (width 0.25) (layer "F.Cu") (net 16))
 (segment (start 156.95 71.92434) (end 156.725 72.14934) (width 0.25) (layer "F.Cu") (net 16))
 (segment (start 156.725 82.495) (end 156.57 82.65) (width 0.25) (layer "F.Cu") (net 16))
 (segment (start 156.725 72.14934) (end 156.725 82.495) (width 0.25) (layer "F.Cu") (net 16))
 (segment (start 156.95 71.92434) (end 156.969838 71.92434) (width 0.25) (layer "F.Cu") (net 16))
 (via (at 156.95 71.92434) (size 0.8) (drill 0.4) (layers "F.Cu" "B.Cu") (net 16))
 (segment (start 156.95 71.92434) (end 156.25616 71.92434) (width 0.25) (layer "B.Cu") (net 16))
 (segment (start 156.25616 71.92434) (end 155.5584 72.6221) (width 0.25) (layer "B.Cu") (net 16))
 (segment (start 155.5584 72.6221) (end 155.5584 73.0375) (width 0.25) (layer "B.Cu") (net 16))
 (segment (start 150.872 76.2) (end 150.872 79.248) (width 0.25) (layer "F.Cu") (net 1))
 (segment (start 151.892 76.2) (end 151.892 79.248) (width 0.25) (layer "F.Cu") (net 2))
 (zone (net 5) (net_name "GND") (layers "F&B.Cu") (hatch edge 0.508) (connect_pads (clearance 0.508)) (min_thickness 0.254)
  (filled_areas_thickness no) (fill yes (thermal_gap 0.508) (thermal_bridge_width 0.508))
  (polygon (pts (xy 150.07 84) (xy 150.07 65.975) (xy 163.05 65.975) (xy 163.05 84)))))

